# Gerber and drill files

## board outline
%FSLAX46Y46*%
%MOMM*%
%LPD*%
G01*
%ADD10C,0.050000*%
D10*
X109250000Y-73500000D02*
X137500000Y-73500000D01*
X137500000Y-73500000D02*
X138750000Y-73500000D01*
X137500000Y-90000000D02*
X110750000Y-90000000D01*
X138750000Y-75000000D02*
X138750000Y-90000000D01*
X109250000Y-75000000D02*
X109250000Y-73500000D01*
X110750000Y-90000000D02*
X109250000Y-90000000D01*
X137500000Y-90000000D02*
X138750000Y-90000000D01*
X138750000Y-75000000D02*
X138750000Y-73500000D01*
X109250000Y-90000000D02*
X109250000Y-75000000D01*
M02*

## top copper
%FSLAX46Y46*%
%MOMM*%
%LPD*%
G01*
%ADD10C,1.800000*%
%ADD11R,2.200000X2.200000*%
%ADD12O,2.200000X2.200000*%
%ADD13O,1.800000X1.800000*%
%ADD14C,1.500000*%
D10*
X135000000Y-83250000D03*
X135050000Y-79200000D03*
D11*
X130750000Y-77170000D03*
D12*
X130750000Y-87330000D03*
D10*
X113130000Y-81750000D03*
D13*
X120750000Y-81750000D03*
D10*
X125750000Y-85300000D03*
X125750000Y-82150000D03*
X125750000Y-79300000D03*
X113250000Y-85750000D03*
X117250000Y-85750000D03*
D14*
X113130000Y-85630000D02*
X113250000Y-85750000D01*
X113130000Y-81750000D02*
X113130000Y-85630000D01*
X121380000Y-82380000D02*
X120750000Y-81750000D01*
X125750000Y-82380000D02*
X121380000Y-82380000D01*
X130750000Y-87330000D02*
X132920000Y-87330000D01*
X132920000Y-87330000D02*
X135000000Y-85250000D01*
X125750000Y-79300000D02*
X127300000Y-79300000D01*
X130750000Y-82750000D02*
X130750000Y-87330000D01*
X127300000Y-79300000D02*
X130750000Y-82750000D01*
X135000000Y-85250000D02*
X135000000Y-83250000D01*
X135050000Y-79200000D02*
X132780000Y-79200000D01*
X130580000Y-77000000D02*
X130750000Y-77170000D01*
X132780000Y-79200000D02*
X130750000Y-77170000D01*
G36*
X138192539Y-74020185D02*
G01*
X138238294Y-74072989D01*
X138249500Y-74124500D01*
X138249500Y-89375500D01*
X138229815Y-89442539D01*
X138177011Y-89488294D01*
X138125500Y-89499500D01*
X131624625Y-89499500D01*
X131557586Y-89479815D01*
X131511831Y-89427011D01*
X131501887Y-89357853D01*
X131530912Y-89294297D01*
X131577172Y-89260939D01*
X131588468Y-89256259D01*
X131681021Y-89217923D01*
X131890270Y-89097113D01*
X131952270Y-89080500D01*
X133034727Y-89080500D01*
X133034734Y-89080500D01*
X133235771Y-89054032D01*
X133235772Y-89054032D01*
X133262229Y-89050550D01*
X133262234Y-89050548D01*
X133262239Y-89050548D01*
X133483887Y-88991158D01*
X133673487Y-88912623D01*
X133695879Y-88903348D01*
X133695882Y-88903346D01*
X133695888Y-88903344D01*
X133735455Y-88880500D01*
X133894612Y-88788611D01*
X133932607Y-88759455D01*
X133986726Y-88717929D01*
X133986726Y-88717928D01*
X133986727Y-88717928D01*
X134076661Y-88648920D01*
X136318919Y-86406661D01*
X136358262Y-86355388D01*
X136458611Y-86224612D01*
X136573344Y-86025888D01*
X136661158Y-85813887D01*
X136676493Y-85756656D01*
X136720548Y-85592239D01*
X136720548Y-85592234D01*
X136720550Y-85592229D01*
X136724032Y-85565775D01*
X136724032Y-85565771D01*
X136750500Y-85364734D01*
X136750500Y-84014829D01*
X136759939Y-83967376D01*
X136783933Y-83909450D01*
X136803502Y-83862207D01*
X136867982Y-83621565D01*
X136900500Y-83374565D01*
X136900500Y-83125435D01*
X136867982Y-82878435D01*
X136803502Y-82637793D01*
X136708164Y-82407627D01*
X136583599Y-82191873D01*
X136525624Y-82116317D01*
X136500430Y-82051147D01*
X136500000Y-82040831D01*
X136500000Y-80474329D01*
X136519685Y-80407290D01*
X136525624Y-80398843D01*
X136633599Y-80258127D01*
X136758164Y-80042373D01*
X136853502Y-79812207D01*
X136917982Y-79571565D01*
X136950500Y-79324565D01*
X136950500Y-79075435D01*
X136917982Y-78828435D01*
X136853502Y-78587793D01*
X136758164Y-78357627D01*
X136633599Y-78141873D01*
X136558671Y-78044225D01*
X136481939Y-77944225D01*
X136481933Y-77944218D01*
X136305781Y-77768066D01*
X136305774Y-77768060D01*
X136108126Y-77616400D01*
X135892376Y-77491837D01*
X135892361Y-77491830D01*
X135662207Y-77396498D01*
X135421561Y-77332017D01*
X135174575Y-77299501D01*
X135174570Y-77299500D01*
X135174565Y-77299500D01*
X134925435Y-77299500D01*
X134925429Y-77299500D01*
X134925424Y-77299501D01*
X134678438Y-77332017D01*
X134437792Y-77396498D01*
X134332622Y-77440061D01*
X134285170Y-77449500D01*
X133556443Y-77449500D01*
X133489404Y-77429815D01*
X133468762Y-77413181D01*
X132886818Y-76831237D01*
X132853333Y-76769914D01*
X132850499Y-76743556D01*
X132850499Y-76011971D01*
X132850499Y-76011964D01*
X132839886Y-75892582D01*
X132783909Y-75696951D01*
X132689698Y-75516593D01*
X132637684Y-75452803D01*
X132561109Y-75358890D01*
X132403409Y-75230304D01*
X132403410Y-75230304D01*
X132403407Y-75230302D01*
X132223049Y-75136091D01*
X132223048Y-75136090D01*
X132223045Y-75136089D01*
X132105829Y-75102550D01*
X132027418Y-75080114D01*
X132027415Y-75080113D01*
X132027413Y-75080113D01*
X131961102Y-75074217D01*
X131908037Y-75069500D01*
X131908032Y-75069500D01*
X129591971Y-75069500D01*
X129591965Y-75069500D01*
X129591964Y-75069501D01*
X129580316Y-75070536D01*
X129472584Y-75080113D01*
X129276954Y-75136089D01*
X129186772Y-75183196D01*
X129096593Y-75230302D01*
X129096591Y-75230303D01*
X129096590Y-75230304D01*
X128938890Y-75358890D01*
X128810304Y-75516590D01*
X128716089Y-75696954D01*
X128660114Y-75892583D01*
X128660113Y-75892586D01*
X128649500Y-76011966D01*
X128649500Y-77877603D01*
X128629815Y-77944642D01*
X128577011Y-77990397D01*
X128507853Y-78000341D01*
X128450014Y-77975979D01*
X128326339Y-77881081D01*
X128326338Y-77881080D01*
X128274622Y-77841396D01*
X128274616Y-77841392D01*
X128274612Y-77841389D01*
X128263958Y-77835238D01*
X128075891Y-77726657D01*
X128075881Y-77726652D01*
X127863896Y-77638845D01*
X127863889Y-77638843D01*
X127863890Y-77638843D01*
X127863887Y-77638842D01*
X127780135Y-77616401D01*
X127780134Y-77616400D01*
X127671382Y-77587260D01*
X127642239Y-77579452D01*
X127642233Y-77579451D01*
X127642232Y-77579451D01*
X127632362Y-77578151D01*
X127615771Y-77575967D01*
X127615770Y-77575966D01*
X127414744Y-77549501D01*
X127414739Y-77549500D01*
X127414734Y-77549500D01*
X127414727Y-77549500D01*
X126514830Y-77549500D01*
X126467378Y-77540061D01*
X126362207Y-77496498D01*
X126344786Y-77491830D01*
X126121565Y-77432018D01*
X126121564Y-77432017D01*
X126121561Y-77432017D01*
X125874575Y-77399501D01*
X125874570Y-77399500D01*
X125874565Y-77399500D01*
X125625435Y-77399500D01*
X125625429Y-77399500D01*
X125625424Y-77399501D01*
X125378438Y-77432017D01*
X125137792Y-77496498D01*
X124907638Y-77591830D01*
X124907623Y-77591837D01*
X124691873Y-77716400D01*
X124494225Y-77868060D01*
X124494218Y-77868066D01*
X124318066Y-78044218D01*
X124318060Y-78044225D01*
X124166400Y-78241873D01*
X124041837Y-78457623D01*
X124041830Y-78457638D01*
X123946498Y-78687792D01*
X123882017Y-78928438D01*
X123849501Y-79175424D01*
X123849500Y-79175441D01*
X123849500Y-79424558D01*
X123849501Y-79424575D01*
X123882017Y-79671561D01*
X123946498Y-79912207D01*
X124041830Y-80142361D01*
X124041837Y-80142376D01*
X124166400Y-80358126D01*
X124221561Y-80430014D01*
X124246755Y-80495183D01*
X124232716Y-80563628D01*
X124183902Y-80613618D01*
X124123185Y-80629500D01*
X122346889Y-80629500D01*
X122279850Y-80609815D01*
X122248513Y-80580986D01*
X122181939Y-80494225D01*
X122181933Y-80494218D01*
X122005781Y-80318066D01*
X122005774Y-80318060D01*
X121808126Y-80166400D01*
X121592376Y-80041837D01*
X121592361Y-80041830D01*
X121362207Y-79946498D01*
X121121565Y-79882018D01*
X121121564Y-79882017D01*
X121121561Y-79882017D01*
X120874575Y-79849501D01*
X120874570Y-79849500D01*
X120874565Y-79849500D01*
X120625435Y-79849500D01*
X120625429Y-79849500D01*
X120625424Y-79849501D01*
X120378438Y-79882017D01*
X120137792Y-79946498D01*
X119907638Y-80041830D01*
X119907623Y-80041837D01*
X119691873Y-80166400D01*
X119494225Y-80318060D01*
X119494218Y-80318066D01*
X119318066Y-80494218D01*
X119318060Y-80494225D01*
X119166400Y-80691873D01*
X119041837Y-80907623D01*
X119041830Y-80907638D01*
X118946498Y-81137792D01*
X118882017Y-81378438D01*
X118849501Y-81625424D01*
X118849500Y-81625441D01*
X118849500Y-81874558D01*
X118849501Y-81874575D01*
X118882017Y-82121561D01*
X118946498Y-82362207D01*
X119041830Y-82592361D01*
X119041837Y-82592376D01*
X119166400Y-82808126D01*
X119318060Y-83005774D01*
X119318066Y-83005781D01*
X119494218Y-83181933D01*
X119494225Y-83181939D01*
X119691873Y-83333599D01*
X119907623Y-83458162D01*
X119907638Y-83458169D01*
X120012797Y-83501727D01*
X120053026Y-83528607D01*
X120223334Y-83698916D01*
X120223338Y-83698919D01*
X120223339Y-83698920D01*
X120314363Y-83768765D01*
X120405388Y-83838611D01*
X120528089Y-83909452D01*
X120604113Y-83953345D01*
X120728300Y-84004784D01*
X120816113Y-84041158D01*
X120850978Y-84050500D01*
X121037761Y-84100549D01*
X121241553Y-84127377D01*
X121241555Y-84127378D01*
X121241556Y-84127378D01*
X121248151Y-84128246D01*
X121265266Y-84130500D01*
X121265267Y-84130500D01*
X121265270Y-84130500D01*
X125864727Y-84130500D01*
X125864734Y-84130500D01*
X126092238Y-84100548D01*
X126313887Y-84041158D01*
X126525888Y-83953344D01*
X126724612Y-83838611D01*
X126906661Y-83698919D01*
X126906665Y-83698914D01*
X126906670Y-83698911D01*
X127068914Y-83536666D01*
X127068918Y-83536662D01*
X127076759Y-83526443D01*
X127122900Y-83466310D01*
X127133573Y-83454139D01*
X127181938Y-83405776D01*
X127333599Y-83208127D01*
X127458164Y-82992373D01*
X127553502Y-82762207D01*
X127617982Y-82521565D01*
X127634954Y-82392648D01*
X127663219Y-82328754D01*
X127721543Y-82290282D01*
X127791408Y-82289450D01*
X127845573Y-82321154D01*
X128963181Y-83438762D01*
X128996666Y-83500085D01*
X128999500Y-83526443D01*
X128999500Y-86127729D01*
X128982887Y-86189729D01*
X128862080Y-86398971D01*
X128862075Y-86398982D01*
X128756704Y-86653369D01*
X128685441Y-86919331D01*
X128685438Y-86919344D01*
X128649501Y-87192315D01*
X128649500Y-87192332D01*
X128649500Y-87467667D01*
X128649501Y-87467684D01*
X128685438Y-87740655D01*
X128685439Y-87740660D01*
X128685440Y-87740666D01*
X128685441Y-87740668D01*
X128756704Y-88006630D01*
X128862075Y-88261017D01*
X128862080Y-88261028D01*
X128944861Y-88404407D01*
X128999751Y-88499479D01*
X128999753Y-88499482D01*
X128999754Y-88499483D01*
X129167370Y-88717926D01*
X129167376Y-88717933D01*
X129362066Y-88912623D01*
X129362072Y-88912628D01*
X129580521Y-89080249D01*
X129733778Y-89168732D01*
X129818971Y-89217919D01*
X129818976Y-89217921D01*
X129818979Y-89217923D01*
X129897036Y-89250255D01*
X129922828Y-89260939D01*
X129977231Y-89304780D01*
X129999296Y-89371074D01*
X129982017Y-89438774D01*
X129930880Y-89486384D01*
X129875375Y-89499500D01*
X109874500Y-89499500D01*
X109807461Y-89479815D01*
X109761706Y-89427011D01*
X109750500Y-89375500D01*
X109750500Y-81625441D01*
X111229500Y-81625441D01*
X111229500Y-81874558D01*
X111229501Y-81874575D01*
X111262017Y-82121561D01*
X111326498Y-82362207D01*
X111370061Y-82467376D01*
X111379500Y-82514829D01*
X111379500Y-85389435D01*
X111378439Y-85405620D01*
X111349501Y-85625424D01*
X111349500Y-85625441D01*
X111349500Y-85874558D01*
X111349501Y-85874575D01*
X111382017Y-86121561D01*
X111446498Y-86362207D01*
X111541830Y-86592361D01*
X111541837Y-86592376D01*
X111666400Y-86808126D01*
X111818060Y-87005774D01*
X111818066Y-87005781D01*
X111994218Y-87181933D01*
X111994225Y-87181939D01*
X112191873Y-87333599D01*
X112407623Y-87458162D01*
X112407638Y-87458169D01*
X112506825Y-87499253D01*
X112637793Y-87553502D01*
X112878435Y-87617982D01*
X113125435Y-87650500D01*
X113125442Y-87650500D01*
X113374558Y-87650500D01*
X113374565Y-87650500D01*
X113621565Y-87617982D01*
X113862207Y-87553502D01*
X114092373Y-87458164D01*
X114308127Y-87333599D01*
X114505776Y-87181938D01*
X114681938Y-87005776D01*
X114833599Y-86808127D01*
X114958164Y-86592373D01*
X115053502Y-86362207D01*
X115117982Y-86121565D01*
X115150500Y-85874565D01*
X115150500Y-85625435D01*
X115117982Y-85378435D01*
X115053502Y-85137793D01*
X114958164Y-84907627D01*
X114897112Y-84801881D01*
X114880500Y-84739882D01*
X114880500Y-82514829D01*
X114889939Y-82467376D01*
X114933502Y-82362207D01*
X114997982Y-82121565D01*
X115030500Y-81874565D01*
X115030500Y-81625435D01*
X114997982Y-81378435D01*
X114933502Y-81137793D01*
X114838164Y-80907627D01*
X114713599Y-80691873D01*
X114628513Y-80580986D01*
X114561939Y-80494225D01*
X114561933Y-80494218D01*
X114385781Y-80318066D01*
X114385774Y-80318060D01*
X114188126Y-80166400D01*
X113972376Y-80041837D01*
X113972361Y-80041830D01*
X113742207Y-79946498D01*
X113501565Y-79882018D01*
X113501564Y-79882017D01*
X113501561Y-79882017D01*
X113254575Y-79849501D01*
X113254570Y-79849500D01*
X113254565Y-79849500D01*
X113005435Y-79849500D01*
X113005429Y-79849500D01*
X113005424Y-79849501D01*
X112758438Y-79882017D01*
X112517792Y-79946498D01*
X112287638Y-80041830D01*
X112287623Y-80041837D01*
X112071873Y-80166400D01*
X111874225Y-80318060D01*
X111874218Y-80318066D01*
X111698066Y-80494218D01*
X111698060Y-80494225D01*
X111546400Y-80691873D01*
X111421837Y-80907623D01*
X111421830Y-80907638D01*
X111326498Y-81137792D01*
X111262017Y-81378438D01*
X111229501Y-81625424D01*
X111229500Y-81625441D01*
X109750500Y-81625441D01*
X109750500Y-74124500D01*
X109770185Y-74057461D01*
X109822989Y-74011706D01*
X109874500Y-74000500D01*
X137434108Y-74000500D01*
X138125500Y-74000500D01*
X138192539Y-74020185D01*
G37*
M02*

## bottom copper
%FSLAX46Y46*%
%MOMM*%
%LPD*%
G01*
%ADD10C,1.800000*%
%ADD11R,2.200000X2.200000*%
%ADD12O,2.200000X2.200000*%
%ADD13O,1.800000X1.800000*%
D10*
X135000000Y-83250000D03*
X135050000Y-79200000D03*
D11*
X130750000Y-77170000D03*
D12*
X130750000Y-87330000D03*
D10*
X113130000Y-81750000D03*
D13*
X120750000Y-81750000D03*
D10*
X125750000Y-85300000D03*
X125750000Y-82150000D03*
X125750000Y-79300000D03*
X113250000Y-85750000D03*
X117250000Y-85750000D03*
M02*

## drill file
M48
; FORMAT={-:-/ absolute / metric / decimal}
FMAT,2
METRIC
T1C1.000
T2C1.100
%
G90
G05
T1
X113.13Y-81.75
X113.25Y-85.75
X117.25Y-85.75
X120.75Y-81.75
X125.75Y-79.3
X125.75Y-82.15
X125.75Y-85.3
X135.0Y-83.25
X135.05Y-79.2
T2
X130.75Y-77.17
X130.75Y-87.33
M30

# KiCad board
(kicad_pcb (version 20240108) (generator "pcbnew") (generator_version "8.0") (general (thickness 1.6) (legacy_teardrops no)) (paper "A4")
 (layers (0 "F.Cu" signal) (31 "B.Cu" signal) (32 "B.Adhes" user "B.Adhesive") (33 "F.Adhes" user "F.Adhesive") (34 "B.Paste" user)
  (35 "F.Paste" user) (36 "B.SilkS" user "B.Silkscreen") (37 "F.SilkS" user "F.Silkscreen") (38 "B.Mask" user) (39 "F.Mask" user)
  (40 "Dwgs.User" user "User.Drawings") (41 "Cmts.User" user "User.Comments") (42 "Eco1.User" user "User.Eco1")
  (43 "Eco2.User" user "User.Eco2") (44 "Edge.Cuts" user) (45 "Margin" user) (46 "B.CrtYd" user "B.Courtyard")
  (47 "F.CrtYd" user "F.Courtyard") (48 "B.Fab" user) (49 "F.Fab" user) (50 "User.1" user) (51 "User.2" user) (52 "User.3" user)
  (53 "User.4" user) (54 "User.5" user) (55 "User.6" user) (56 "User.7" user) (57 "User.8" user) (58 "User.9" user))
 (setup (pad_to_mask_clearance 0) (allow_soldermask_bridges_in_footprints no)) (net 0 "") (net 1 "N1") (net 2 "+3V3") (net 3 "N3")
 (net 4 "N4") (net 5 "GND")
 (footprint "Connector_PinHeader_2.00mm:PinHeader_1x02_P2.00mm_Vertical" (layer "F.Cu") (at 135 83.25 180)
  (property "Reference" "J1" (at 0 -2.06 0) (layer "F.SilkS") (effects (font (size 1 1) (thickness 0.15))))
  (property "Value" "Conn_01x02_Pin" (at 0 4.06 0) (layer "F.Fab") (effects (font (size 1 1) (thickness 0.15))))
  (pad "1" thru_hole circle (at 0 0 180) (size 1.8 1.8) (drill 1) (layers "*.Cu" "*.Mask") (remove_unused_layers no) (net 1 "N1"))
  (pad "2" thru_hole circle (at -0.05 4.05 180) (size 1.8 1.8) (drill 1) (layers "*.Cu" "*.Mask") (remove_unused_layers no) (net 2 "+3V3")))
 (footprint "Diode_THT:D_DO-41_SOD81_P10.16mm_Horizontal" (layer "F.Cu") (at 130.75 77.17 -90)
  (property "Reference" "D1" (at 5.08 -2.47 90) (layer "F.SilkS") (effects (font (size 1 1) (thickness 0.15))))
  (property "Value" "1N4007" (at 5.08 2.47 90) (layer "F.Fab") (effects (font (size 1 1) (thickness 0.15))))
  (pad "1" thru_hole rect (at 0 0 270) (size 2.2 2.2) (drill 1.1) (layers "*.Cu" "*.Mask") (remove_unused_layers no) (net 2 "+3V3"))
  (pad "2" thru_hole oval (at 10.16 0 270) (size 2.2 2.2) (drill 1.1) (layers "*.Cu" "*.Mask") (remove_unused_layers no) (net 1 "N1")))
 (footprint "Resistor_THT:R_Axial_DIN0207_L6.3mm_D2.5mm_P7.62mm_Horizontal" (layer "F.Cu") (at 113.13 81.75)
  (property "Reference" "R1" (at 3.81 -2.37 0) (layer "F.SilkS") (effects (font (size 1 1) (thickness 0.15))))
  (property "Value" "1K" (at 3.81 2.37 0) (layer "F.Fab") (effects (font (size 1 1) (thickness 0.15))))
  (pad "1" thru_hole circle (at 0 0) (size 1.8 1.8) (drill 1) (layers "*.Cu" "*.Mask") (remove_unused_layers no) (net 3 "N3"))
  (pad "2" thru_hole oval (at 7.62 0) (size 1.8 1.8) (drill 1) (layers "*.Cu" "*.Mask") (remove_unused_layers no) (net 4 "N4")))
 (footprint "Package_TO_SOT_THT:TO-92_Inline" (layer "F.Cu") (at 125.75 83.65 90)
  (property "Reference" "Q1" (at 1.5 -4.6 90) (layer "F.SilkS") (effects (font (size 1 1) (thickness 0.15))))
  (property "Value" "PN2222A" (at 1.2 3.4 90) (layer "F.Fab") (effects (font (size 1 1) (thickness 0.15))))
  (pad "1" thru_hole circle (at -1.65 0 90) (size 1.8 1.8) (drill 1) (layers "*.Cu" "*.Mask") (remove_unused_layers no) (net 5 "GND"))
  (pad "2" thru_hole circle (at 1.5 0 90) (size 1.8 1.8) (drill 1) (layers "*.Cu" "*.Mask") (remove_unused_layers no) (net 4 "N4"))
  (pad "3" thru_hole circle (at 4.35 0 90) (size 1.8 1.8) (drill 1) (layers "*.Cu" "*.Mask") (remove_unused_layers no) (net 1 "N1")))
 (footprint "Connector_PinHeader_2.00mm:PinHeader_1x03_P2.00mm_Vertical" (layer "F.Cu") (at 113.25 85.75 90)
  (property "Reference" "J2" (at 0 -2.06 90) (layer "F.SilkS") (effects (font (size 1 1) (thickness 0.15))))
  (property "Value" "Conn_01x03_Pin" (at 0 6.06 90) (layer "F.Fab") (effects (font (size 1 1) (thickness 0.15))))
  (pad "1" thru_hole circle (at 0 0 90) (size 1.8 1.8) (drill 1) (layers "*.Cu" "*.Mask") (remove_unused_layers no) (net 3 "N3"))
  (pad "3" thru_hole circle (at 0 4 90) (size 1.8 1.8) (drill 1) (layers "*.Cu" "*.Mask") (remove_unused_layers no) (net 5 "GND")))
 (gr_line (start 109.25 73.5) (end 137.5 73.5) (stroke (width 0.05) (type default)) (layer "Edge.Cuts"))
 (gr_line (start 137.5 73.5) (end 138.75 73.5) (stroke (width 0.05) (type default)) (layer "Edge.Cuts"))
 (gr_line (start 137.5 90) (end 110.75 90) (stroke (width 0.05) (type default)) (layer "Edge.Cuts"))
 (gr_line (start 138.75 75) (end 138.75 90) (stroke (width 0.05) (type default)) (layer "Edge.Cuts"))
 (gr_line (start 109.25 75) (end 109.25 73.5) (stroke (width 0.05) (type default)) (layer "Edge.Cuts"))
 (gr_line (start 110.75 90) (end 109.25 90) (stroke (width 0.05) (type default)) (layer "Edge.Cuts"))
 (gr_line (start 137.5 90) (end 138.75 90) (stroke (width 0.05) (type default)) (layer "Edge.Cuts"))
 (gr_line (start 138.75 75) (end 138.75 73.5) (stroke (width 0.05) (type default)) (layer "Edge.Cuts"))
 (gr_line (start 109.25 90) (end 109.25 75) (stroke (width 0.05) (type default)) (layer "Edge.Cuts"))
 (segment (start 113.13 85.63) (end 113.25 85.75) (width 1.5) (layer "F.Cu") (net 3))
 (segment (start 113.13 81.75) (end 113.13 85.63) (width 1.5) (layer "F.Cu") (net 3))
 (segment (start 121.38 82.38) (end 120.75 81.75) (width 1.5) (layer "F.Cu") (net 4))
 (segment (start 125.75 82.38) (end 121.38 82.38) (width 1.5) (layer "F.Cu") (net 4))
 (segment (start 130.75 87.33) (end 132.92 87.33) (width 1.5) (layer "F.Cu") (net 1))
 (segment (start 132.92 87.33) (end 135 85.25) (width 1.5) (layer "F.Cu") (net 1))
 (segment (start 125.75 79.3) (end 127.3 79.3) (width 1.5) (layer "F.Cu") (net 1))
 (segment (start 130.75 82.75) (end 130.75 87.33) (width 1.5) (layer "F.Cu") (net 1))
 (segment (start 127.3 79.3) (end 130.75 82.75) (width 1.5) (layer "F.Cu") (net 1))
 (segment (start 135 85.25) (end 135 83.25) (width 1.5) (layer "F.Cu") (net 1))
 (segment (start 135.05 79.2) (end 132.78 79.2) (width 1.5) (layer "F.Cu") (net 2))
 (segment (start 130.58 77) (end 130.75 77.17) (width 1.5) (layer "F.Cu") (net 2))
 (segment (start 132.78 79.2) (end 130.75 77.17) (width 1.5) (layer "F.Cu") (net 2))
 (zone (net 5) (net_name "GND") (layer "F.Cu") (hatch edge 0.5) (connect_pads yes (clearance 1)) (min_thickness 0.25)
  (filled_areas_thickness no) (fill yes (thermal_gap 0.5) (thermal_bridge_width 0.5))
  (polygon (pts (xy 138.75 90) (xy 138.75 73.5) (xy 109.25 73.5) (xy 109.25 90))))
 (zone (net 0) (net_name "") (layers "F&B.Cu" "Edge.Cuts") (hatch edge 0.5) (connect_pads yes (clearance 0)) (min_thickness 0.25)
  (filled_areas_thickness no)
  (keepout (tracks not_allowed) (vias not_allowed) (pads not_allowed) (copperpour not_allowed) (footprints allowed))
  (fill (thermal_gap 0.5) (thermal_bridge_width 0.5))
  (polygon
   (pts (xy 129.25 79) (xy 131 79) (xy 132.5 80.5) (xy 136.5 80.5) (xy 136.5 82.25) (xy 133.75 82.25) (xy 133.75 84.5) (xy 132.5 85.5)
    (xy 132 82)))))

